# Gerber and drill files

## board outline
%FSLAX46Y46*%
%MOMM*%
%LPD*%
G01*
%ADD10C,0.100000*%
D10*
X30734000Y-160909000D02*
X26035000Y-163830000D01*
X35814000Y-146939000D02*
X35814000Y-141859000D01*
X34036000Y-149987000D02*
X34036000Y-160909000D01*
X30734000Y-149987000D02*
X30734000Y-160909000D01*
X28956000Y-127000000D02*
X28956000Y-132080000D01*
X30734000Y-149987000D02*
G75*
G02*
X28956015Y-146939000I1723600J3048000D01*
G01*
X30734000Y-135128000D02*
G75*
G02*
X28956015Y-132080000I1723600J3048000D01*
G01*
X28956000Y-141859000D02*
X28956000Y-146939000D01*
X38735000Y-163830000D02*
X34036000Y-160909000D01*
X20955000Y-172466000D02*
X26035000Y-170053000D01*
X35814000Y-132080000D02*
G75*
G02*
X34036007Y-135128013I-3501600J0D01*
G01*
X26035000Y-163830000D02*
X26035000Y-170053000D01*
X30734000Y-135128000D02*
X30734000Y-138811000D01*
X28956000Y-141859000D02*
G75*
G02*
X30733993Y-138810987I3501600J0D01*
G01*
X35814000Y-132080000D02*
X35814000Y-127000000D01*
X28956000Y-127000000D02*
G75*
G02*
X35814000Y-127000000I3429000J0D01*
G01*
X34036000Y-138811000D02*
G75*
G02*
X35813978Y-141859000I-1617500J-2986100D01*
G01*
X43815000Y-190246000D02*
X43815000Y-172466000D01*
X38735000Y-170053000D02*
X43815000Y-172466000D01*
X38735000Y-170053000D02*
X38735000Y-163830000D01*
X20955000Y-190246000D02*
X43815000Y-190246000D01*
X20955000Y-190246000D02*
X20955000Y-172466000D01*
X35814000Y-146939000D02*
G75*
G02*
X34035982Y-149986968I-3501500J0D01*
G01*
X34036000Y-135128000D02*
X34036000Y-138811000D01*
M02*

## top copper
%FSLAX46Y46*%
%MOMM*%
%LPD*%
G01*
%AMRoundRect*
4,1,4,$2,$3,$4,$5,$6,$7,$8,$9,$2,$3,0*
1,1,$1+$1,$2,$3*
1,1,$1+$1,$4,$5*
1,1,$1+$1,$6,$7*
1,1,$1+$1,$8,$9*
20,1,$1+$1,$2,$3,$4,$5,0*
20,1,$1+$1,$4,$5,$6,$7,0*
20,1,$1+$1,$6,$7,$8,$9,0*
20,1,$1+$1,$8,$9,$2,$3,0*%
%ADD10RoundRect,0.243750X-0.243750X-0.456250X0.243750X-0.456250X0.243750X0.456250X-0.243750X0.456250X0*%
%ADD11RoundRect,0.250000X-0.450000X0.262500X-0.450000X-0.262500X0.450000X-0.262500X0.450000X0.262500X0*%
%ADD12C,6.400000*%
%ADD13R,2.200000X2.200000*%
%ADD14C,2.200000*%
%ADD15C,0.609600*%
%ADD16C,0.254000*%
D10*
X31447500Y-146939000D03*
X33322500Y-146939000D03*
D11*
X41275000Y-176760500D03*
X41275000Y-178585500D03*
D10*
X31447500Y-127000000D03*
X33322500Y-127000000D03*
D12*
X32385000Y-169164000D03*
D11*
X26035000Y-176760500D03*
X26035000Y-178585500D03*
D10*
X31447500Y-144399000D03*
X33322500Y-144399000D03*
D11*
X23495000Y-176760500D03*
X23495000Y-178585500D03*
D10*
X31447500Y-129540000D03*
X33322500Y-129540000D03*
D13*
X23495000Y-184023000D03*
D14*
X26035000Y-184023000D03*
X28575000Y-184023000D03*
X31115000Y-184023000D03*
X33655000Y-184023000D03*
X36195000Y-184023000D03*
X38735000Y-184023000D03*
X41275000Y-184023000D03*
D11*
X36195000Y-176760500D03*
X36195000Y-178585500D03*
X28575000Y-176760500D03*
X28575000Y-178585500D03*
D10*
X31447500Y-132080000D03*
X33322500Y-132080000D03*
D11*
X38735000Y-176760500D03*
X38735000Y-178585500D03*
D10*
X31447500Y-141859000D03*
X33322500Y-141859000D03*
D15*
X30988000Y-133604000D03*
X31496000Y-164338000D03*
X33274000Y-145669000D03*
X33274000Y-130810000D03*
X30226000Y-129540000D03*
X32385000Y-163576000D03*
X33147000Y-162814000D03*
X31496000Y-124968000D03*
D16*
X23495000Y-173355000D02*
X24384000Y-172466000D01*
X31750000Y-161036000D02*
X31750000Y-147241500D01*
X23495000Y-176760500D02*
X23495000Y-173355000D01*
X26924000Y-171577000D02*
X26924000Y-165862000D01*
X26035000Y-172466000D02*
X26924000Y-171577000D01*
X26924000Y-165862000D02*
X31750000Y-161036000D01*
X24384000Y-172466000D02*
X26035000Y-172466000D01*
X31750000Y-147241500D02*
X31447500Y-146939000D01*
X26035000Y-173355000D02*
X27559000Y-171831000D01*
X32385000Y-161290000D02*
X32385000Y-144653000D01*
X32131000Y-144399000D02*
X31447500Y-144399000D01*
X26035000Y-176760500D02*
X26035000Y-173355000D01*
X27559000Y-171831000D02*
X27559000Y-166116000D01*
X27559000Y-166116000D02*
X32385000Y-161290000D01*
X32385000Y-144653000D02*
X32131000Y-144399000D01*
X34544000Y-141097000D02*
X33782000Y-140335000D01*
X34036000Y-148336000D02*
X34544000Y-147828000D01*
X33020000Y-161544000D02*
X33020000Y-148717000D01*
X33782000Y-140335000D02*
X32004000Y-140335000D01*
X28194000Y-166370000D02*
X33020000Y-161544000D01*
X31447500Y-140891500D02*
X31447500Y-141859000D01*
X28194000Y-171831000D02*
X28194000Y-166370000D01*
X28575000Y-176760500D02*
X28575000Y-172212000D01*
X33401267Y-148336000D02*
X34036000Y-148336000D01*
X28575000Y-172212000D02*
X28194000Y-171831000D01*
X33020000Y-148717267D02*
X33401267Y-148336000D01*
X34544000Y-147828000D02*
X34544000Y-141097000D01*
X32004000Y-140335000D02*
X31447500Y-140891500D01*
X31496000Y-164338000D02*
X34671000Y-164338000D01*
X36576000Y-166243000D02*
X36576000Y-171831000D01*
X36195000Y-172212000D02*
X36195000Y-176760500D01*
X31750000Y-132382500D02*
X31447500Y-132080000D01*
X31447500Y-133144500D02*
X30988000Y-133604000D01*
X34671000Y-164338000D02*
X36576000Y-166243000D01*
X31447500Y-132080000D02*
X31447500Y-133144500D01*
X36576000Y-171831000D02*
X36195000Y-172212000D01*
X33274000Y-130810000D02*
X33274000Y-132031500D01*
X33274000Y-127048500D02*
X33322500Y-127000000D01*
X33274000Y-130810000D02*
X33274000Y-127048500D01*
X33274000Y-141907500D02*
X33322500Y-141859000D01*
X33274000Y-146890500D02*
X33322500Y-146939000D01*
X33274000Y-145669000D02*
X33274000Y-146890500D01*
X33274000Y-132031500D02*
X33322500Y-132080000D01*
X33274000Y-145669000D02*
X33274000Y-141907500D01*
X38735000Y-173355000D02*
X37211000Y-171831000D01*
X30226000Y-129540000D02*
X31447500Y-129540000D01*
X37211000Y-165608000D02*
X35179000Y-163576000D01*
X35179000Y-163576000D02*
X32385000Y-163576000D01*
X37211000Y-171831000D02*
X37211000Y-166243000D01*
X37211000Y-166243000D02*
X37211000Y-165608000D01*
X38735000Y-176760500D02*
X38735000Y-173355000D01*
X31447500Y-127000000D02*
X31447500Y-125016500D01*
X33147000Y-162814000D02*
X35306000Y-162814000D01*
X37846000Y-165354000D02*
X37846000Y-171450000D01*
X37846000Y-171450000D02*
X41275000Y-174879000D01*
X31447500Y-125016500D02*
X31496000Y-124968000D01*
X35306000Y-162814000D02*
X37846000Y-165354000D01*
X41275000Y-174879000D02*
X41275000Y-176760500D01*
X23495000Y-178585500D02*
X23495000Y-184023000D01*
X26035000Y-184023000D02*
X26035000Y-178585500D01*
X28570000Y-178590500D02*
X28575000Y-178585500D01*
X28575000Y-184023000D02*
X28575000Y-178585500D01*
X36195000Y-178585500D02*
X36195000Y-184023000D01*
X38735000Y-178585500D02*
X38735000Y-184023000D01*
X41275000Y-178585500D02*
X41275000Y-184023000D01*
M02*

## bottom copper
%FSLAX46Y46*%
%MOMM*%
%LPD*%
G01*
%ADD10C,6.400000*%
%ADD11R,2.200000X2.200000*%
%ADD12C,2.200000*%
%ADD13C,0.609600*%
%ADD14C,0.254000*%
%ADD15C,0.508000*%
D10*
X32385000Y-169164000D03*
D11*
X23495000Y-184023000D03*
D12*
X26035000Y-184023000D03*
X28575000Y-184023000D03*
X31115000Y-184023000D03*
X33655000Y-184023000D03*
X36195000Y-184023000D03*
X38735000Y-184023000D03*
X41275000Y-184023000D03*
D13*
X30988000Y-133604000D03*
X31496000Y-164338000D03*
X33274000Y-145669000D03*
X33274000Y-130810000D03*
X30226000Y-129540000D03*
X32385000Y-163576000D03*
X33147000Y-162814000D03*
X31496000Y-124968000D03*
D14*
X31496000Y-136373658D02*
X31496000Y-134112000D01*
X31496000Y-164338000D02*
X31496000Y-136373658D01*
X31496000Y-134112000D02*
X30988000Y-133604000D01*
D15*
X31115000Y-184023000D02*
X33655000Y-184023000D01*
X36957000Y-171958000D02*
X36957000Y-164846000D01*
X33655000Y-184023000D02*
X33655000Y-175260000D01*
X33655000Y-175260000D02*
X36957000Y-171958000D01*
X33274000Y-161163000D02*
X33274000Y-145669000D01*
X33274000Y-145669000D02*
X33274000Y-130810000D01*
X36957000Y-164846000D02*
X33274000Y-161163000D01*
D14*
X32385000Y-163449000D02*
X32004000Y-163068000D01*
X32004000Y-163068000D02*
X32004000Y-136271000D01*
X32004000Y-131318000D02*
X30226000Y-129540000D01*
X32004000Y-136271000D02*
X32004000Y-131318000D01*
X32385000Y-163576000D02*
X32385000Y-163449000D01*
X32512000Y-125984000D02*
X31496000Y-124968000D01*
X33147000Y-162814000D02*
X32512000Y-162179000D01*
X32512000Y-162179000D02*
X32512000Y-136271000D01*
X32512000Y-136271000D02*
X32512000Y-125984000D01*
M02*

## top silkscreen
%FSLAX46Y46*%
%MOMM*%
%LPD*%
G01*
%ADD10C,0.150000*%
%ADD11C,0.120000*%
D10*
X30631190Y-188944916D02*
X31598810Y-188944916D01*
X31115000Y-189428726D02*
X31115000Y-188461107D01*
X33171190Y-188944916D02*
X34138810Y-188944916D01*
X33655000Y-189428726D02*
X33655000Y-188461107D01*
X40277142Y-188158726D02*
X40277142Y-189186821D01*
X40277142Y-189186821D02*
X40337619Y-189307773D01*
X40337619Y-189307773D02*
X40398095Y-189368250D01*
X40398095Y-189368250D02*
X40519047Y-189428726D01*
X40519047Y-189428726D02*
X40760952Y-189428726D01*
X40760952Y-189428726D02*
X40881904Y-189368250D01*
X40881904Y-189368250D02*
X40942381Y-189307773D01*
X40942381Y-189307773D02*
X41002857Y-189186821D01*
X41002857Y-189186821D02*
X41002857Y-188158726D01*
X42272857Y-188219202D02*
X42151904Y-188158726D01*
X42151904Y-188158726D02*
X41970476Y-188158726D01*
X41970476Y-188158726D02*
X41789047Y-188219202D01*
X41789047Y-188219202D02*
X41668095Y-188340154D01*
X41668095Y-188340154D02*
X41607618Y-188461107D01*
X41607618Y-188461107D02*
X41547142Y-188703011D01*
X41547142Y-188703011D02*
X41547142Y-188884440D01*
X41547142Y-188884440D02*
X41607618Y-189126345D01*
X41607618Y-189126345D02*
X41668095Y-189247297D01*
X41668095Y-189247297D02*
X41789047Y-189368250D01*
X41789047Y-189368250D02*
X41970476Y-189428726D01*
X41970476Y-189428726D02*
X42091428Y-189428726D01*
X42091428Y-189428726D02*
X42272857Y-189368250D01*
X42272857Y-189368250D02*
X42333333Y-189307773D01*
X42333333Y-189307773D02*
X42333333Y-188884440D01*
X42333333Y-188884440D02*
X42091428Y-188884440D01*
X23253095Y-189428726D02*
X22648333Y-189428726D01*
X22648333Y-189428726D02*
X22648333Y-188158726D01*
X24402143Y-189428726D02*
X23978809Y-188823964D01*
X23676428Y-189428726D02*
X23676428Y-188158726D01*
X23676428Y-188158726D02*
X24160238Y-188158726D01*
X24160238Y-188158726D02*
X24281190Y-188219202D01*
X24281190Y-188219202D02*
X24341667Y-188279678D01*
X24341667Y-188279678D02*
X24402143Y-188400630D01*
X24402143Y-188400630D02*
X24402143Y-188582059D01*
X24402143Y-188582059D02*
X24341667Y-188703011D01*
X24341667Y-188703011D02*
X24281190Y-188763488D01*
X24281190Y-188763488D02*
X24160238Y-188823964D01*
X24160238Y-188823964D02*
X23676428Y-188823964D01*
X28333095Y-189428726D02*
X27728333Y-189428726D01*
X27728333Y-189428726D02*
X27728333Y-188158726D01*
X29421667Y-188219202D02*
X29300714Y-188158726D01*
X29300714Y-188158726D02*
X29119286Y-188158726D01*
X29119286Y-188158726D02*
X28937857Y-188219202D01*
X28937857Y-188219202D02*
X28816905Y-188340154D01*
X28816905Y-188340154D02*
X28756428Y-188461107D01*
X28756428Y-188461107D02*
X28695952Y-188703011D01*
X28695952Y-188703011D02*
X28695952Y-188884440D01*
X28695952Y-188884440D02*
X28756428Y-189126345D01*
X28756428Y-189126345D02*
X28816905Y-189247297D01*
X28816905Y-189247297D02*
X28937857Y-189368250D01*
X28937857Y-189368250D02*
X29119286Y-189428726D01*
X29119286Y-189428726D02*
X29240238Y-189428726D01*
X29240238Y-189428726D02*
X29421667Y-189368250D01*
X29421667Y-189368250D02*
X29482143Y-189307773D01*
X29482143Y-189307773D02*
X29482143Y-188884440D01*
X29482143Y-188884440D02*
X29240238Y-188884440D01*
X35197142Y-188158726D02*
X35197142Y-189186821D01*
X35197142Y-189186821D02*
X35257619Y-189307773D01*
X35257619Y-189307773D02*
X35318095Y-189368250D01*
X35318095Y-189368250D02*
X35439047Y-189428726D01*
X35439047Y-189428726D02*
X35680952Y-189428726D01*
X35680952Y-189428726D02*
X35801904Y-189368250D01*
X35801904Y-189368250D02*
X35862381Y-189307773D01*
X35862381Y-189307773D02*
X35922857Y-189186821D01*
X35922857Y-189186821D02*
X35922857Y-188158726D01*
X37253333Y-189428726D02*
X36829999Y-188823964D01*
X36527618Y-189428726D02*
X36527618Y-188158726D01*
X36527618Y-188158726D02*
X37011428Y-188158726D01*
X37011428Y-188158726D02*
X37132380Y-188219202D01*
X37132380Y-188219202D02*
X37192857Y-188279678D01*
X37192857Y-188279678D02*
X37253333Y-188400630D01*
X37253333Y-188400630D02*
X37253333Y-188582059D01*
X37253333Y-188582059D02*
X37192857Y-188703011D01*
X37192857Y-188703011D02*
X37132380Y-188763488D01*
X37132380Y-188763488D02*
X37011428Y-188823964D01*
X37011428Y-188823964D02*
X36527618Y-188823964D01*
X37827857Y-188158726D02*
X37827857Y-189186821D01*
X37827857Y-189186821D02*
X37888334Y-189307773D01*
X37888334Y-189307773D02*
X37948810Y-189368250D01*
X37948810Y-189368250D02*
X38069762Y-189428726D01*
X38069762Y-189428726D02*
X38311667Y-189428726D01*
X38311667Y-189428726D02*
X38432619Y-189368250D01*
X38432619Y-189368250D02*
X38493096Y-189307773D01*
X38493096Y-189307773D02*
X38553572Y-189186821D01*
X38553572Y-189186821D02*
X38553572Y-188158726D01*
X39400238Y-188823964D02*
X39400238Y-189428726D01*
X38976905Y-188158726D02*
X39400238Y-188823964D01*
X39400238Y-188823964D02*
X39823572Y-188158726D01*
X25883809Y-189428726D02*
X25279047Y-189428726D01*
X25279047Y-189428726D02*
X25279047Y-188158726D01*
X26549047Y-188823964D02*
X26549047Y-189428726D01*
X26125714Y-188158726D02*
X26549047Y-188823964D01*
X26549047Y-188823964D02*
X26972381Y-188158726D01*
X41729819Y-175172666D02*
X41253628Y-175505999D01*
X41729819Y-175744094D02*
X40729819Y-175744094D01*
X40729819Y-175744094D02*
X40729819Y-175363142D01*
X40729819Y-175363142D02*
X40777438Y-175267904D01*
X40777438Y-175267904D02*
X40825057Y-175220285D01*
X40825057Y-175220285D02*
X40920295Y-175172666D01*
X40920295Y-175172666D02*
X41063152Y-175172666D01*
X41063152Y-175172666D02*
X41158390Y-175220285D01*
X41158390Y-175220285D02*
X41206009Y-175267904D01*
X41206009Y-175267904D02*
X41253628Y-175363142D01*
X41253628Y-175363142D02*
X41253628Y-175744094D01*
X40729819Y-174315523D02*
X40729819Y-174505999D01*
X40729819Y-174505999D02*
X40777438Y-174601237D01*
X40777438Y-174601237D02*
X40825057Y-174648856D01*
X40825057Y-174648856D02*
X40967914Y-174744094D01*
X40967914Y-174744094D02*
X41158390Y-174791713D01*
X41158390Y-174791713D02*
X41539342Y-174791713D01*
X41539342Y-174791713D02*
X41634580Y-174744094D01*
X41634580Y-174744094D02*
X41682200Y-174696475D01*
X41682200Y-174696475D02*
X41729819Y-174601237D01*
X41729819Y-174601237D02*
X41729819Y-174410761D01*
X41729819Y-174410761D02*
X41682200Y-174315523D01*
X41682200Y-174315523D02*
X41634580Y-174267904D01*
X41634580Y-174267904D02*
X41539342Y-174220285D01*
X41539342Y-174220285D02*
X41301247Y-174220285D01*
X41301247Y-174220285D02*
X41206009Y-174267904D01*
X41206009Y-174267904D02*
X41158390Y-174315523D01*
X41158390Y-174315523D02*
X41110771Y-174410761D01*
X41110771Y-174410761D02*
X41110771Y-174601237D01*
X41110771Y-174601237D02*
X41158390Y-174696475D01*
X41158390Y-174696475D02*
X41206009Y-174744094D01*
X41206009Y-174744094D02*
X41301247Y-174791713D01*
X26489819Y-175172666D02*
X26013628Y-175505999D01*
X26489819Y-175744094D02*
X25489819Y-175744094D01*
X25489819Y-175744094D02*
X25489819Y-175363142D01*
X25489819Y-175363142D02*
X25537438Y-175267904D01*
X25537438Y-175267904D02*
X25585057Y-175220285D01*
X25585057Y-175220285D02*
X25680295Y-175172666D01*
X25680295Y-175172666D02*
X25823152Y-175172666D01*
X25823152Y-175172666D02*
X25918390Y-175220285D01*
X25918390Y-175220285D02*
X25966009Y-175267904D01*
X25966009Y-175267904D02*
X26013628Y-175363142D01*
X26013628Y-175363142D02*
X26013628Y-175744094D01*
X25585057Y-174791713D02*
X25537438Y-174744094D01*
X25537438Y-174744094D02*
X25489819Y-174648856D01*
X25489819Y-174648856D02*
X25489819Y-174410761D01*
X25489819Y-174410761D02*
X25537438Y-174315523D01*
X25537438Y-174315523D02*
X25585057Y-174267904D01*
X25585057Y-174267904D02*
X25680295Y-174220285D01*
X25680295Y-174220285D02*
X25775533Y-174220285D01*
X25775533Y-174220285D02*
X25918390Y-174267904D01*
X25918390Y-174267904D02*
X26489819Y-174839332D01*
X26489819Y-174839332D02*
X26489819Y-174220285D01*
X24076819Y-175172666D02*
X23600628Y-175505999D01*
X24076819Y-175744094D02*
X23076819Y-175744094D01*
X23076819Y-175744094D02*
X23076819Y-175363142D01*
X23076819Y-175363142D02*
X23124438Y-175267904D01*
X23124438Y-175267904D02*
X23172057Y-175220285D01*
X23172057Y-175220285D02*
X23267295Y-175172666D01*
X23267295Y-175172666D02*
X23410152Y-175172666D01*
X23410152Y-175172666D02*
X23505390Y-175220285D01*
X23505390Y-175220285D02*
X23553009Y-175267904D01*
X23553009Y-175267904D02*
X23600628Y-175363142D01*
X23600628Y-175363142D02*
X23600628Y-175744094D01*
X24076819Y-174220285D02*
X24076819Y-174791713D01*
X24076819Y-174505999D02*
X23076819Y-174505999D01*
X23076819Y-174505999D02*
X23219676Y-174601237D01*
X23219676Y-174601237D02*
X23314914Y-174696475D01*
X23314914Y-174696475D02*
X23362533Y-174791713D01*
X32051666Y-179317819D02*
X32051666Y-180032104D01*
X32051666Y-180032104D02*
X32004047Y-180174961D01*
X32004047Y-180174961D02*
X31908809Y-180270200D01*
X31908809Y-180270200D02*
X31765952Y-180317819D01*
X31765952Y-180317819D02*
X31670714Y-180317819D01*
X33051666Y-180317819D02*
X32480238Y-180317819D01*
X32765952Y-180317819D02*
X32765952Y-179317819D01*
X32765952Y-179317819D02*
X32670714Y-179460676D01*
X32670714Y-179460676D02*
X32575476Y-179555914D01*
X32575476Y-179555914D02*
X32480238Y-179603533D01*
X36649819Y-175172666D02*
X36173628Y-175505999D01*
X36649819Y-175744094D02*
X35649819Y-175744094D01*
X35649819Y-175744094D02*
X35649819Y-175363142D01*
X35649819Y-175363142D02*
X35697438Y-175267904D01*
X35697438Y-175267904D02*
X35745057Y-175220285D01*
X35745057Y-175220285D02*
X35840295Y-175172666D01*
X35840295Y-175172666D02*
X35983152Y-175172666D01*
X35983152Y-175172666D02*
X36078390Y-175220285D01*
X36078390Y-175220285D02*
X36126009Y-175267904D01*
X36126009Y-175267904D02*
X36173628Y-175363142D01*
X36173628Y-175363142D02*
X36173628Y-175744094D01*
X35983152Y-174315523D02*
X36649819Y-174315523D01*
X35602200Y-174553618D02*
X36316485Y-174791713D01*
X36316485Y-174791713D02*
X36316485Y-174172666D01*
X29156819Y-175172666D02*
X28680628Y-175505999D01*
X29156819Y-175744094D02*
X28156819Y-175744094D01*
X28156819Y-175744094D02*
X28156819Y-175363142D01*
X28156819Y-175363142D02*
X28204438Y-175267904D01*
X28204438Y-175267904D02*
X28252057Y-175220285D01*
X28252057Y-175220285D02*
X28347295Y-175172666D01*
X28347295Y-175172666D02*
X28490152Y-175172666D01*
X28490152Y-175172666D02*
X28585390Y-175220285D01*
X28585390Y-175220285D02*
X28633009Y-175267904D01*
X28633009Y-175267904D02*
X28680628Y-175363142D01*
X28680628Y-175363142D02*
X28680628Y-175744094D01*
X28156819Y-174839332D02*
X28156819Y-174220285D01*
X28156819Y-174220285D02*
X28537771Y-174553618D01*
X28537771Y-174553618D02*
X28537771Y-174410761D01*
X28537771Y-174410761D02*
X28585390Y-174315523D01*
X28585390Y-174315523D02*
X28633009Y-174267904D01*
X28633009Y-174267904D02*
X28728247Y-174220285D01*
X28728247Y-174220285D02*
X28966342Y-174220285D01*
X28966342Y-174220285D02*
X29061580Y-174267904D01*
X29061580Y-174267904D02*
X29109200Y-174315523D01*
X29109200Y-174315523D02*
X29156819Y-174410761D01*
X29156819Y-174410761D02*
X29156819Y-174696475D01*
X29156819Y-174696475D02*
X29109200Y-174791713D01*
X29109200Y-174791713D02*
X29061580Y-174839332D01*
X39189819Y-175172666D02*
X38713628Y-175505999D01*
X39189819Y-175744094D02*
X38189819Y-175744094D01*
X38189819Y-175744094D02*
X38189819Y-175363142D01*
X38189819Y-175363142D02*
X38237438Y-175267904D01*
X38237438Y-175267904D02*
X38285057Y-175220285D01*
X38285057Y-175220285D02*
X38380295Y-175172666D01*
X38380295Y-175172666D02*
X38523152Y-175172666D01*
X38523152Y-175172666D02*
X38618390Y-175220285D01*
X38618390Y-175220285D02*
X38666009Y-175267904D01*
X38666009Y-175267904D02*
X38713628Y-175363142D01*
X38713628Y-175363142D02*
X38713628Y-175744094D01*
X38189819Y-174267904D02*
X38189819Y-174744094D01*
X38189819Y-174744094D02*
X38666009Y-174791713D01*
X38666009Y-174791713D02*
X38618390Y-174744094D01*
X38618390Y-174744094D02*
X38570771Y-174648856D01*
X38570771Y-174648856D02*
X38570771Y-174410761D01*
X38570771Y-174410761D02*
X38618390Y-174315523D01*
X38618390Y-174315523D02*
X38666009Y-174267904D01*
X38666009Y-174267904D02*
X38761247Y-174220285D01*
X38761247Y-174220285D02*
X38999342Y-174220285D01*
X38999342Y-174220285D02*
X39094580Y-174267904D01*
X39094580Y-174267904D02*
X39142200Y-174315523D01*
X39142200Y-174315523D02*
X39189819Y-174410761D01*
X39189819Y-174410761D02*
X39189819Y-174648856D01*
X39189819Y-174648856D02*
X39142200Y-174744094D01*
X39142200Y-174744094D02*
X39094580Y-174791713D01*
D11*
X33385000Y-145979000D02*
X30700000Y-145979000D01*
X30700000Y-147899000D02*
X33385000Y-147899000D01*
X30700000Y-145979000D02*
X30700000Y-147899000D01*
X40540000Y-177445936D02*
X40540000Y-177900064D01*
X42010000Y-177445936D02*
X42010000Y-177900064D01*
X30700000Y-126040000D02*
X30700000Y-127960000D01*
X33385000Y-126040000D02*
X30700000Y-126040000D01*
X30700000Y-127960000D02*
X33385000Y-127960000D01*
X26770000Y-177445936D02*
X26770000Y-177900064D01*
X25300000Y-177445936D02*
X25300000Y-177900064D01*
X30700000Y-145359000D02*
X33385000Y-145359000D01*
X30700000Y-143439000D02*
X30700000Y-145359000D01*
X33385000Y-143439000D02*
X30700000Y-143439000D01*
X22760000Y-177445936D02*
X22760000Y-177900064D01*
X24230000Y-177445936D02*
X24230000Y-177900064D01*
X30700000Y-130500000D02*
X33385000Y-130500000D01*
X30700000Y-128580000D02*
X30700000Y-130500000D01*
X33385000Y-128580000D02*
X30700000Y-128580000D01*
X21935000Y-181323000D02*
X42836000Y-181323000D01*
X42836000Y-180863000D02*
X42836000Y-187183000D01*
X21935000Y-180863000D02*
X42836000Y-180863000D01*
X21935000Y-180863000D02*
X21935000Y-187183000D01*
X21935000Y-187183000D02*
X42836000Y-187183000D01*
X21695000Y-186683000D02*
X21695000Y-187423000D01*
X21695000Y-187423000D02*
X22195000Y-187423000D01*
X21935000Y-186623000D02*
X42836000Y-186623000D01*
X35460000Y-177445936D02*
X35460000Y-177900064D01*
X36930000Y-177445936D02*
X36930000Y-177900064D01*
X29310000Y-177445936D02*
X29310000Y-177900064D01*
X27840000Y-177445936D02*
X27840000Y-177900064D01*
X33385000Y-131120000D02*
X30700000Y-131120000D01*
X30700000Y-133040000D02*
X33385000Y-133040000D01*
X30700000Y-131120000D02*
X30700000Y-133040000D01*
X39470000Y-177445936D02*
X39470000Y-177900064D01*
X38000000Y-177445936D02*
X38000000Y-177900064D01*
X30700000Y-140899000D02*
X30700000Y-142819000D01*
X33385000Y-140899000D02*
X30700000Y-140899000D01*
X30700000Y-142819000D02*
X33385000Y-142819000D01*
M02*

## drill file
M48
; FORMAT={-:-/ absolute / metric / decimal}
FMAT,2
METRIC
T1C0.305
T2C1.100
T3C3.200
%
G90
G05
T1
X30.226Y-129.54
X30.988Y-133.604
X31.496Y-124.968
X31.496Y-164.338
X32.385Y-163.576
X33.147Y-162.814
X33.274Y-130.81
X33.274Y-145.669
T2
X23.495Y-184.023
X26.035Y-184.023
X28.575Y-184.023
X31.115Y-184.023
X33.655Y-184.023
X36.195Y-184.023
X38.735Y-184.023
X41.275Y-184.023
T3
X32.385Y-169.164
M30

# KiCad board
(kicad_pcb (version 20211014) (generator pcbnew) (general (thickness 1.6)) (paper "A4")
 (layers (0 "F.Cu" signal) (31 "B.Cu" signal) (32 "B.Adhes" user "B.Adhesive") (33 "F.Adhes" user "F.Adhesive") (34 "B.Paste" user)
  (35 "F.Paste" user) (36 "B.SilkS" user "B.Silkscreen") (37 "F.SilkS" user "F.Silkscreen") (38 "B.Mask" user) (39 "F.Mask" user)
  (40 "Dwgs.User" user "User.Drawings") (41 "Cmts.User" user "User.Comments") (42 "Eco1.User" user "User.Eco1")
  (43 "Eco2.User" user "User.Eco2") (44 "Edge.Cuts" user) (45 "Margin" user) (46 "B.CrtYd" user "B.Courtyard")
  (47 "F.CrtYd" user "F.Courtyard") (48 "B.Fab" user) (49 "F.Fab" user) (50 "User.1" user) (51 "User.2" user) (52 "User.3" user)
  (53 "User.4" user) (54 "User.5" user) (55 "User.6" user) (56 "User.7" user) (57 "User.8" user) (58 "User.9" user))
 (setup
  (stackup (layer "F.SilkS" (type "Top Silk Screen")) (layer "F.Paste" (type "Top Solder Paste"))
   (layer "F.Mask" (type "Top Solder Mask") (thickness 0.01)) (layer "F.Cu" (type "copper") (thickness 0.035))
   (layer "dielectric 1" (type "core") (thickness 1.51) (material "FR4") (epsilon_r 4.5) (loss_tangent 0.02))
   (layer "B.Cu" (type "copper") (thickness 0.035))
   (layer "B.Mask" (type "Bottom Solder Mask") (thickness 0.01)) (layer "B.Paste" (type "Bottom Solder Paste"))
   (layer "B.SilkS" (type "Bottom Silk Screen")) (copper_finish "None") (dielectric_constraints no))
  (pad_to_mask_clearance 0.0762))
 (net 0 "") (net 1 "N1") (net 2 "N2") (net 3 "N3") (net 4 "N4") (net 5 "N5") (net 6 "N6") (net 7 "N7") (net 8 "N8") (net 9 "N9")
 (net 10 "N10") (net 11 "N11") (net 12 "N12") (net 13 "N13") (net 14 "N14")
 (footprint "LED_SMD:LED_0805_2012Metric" (layer "F.Cu") (at 32.385 146.939)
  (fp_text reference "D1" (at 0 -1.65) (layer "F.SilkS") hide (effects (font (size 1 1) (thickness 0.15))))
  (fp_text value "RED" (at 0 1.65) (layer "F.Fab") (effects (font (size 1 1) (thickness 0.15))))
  (fp_line (start 1 -0.96) (end -1.685 -0.96) (layer "F.SilkS") (width 0.12))
  (fp_line (start -1.685 0.96) (end 1 0.96) (layer "F.SilkS") (width 0.12))
  (fp_line (start -1.685 -0.96) (end -1.685 0.96) (layer "F.SilkS") (width 0.12))
  (pad "1" smd roundrect (at -0.9375 0) (size 0.975 1.4) (layers "F.Cu" "F.Paste" "F.Mask") (roundrect_rratio 0.25) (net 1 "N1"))
  (pad "2" smd roundrect (at 0.9375 0) (size 0.975 1.4) (layers "F.Cu" "F.Paste" "F.Mask") (roundrect_rratio 0.25) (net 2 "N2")))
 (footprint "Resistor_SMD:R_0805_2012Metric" (layer "F.Cu") (at 41.275 177.673 -90)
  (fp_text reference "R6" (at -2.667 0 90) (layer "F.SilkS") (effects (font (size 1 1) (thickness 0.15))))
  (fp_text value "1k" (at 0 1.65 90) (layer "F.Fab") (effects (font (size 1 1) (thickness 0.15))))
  (fp_line (start -0.227064 0.735) (end 0.227064 0.735) (layer "F.SilkS") (width 0.12))
  (fp_line (start -0.227064 -0.735) (end 0.227064 -0.735) (layer "F.SilkS") (width 0.12))
  (pad "1" smd roundrect (at -0.9125 0 270) (size 1.025 1.4) (layers "F.Cu" "F.Paste" "F.Mask") (roundrect_rratio 0.243902) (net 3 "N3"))
  (pad "2" smd roundrect (at 0.9125 0 270) (size 1.025 1.4) (layers "F.Cu" "F.Paste" "F.Mask") (roundrect_rratio 0.243902) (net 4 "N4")))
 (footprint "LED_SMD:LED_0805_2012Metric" (layer "F.Cu") (at 32.385 127)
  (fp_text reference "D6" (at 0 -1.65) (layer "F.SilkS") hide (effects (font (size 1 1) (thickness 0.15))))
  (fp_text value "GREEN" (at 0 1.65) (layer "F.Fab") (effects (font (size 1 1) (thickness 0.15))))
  (fp_line (start -1.685 -0.96) (end -1.685 0.96) (layer "F.SilkS") (width 0.12))
  (fp_line (start 1 -0.96) (end -1.685 -0.96) (layer "F.SilkS") (width 0.12))
  (fp_line (start -1.685 0.96) (end 1 0.96) (layer "F.SilkS") (width 0.12))
  (pad "1" smd roundrect (at -0.9375 0) (size 0.975 1.4) (layers "F.Cu" "F.Paste" "F.Mask") (roundrect_rratio 0.25) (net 3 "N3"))
  (pad "2" smd roundrect (at 0.9375 0) (size 0.975 1.4) (layers "F.Cu" "F.Paste" "F.Mask") (roundrect_rratio 0.25) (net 2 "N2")))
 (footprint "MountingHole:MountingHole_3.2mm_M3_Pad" (layer "F.Cu") (at 32.385 169.164) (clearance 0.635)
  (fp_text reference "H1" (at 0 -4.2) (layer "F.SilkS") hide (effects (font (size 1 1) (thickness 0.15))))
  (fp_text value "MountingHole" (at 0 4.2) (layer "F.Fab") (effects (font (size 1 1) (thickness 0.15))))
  (pad "1" thru_hole circle (at 0 0) (size 6.4 6.4) (drill 3.2) (layers *.Cu *.Mask) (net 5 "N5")))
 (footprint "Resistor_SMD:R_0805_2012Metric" (layer "F.Cu") (at 26.035 177.673 -90)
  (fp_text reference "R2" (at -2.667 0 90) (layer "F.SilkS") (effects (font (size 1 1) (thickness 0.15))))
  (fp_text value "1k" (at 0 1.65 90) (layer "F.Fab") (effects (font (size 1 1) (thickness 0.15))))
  (fp_line (start -0.227064 -0.735) (end 0.227064 -0.735) (layer "F.SilkS") (width 0.12))
  (fp_line (start -0.227064 0.735) (end 0.227064 0.735) (layer "F.SilkS") (width 0.12))
  (pad "1" smd roundrect (at -0.9125 0 270) (size 1.025 1.4) (layers "F.Cu" "F.Paste" "F.Mask") (roundrect_rratio 0.243902) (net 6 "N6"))
  (pad "2" smd roundrect (at 0.9125 0 270) (size 1.025 1.4) (layers "F.Cu" "F.Paste" "F.Mask") (roundrect_rratio 0.243902) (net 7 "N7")))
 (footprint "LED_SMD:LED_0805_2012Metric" (layer "F.Cu") (at 32.385 144.399)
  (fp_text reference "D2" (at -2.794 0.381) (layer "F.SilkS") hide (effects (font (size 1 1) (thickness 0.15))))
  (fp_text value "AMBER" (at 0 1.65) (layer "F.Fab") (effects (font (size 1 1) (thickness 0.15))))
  (fp_line (start -1.685 0.96) (end 1 0.96) (layer "F.SilkS") (width 0.12))
  (fp_line (start -1.685 -0.96) (end -1.685 0.96) (layer "F.SilkS") (width 0.12))
  (fp_line (start 1 -0.96) (end -1.685 -0.96) (layer "F.SilkS") (width 0.12))
  (pad "1" smd roundrect (at -0.9375 0) (size 0.975 1.4) (layers "F.Cu" "F.Paste" "F.Mask") (roundrect_rratio 0.25) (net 6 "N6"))
  (pad "2" smd roundrect (at 0.9375 0) (size 0.975 1.4) (layers "F.Cu" "F.Paste" "F.Mask") (roundrect_rratio 0.25) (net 2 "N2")))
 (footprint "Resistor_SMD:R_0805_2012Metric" (layer "F.Cu") (at 23.495 177.673 -90)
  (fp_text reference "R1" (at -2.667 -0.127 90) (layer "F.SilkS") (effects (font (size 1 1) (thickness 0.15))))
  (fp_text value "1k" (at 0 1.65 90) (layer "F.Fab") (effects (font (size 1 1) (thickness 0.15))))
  (fp_line (start -0.227064 0.735) (end 0.227064 0.735) (layer "F.SilkS") (width 0.12))
  (fp_line (start -0.227064 -0.735) (end 0.227064 -0.735) (layer "F.SilkS") (width 0.12))
  (pad "1" smd roundrect (at -0.9125 0 270) (size 1.025 1.4) (layers "F.Cu" "F.Paste" "F.Mask") (roundrect_rratio 0.243902) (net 1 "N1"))
  (pad "2" smd roundrect (at 0.9125 0 270) (size 1.025 1.4) (layers "F.Cu" "F.Paste" "F.Mask") (roundrect_rratio 0.243902) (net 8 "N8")))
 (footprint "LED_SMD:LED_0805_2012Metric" (layer "F.Cu") (at 32.385 129.54)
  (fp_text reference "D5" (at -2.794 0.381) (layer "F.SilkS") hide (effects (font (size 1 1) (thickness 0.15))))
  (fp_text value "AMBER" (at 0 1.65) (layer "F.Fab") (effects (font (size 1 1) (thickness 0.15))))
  (fp_line (start -1.685 0.96) (end 1 0.96) (layer "F.SilkS") (width 0.12))
  (fp_line (start -1.685 -0.96) (end -1.685 0.96) (layer "F.SilkS") (width 0.12))
  (fp_line (start 1 -0.96) (end -1.685 -0.96) (layer "F.SilkS") (width 0.12))
  (pad "1" smd roundrect (at -0.9375 0) (size 0.975 1.4) (layers "F.Cu" "F.Paste" "F.Mask") (roundrect_rratio 0.25) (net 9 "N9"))
  (pad "2" smd roundrect (at 0.9375 0) (size 0.975 1.4) (layers "F.Cu" "F.Paste" "F.Mask") (roundrect_rratio 0.25) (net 2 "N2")))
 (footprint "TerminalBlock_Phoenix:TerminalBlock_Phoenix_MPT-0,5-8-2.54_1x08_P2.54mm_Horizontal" (layer "F.Cu") (at 23.495 184.023)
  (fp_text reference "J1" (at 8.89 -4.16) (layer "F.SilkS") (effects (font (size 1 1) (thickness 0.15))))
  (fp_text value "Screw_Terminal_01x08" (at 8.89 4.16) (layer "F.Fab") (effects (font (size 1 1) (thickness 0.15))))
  (fp_line (start -1.56 -2.7) (end 19.341 -2.7) (layer "F.SilkS") (width 0.12))
  (fp_line (start 19.341 -3.16) (end 19.341 3.16) (layer "F.SilkS") (width 0.12))
  (fp_line (start -1.56 -3.16) (end 19.341 -3.16) (layer "F.SilkS") (width 0.12))
  (fp_line (start -1.56 -3.16) (end -1.56 3.16) (layer "F.SilkS") (width 0.12))
  (fp_line (start -1.56 3.16) (end 19.341 3.16) (layer "F.SilkS") (width 0.12))
  (fp_line (start -1.8 2.66) (end -1.8 3.4) (layer "F.SilkS") (width 0.12))
  (fp_line (start -1.8 3.4) (end -1.3 3.4) (layer "F.SilkS") (width 0.12))
  (fp_line (start -1.56 2.6) (end 19.341 2.6) (layer "F.SilkS") (width 0.12))
  (pad "1" thru_hole rect (at 0 0) (size 2.2 2.2) (drill 1.1) (layers F&B.Cu *.Mask) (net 8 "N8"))
  (pad "2" thru_hole circle (at 2.54 0) (size 2.2 2.2) (drill 1.1) (layers F&B.Cu *.Mask) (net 7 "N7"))
  (pad "3" thru_hole circle (at 5.08 0) (size 2.2 2.2) (drill 1.1) (layers F&B.Cu *.Mask) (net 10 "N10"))
  (pad "4" thru_hole circle (at 7.62 0) (size 2.2 2.2) (drill 1.1) (layers F&B.Cu *.Mask) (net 2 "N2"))
  (pad "5" thru_hole circle (at 10.16 0) (size 2.2 2.2) (drill 1.1) (layers F&B.Cu *.Mask) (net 2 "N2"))
  (pad "6" thru_hole circle (at 12.7 0) (size 2.2 2.2) (drill 1.1) (layers F&B.Cu *.Mask) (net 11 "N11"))
  (pad "7" thru_hole circle (at 15.24 0) (size 2.2 2.2) (drill 1.1) (layers F&B.Cu *.Mask) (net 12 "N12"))
  (pad "8" thru_hole circle (at 17.78 0) (size 2.2 2.2) (drill 1.1) (layers F&B.Cu *.Mask) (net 4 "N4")))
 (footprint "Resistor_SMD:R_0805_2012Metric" (layer "F.Cu") (at 36.195 177.673 -90)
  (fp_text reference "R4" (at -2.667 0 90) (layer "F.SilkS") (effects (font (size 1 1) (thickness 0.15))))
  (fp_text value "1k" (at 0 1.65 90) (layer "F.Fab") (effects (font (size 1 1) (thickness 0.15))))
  (fp_line (start -0.227064 0.735) (end 0.227064 0.735) (layer "F.SilkS") (width 0.12))
  (fp_line (start -0.227064 -0.735) (end 0.227064 -0.735) (layer "F.SilkS") (width 0.12))
  (pad "1" smd roundrect (at -0.9125 0 270) (size 1.025 1.4) (layers "F.Cu" "F.Paste" "F.Mask") (roundrect_rratio 0.243902) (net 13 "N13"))
  (pad "2" smd roundrect (at 0.9125 0 270) (size 1.025 1.4) (layers "F.Cu" "F.Paste" "F.Mask") (roundrect_rratio 0.243902) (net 11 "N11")))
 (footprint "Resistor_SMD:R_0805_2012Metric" (layer "F.Cu") (at 28.575 177.673 -90)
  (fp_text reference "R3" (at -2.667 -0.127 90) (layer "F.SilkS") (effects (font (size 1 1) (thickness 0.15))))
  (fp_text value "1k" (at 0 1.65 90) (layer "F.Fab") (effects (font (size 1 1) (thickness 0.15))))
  (fp_line (start -0.227064 -0.735) (end 0.227064 -0.735) (layer "F.SilkS") (width 0.12))
  (fp_line (start -0.227064 0.735) (end 0.227064 0.735) (layer "F.SilkS") (width 0.12))
  (pad "1" smd roundrect (at -0.9125 0 270) (size 1.025 1.4) (layers "F.Cu" "F.Paste" "F.Mask") (roundrect_rratio 0.243902) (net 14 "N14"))
  (pad "2" smd roundrect (at 0.9125 0 270) (size 1.025 1.4) (layers "F.Cu" "F.Paste" "F.Mask") (roundrect_rratio 0.243902) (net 10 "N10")))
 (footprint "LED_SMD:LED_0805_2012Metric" (layer "F.Cu") (at 32.385 132.08)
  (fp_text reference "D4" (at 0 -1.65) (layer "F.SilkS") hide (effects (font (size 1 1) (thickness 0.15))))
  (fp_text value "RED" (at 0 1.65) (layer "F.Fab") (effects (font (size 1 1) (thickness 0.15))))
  (fp_line (start 1 -0.96) (end -1.685 -0.96) (layer "F.SilkS") (width 0.12))
  (fp_line (start -1.685 0.96) (end 1 0.96) (layer "F.SilkS") (width 0.12))
  (fp_line (start -1.685 -0.96) (end -1.685 0.96) (layer "F.SilkS") (width 0.12))
  (pad "1" smd roundrect (at -0.9375 0) (size 0.975 1.4) (layers "F.Cu" "F.Paste" "F.Mask") (roundrect_rratio 0.25) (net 13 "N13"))
  (pad "2" smd roundrect (at 0.9375 0) (size 0.975 1.4) (layers "F.Cu" "F.Paste" "F.Mask") (roundrect_rratio 0.25) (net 2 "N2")))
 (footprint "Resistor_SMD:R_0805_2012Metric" (layer "F.Cu") (at 38.735 177.673 -90)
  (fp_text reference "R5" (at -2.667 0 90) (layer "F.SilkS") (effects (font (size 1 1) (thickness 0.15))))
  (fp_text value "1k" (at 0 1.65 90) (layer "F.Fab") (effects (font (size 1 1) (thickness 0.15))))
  (fp_line (start -0.227064 -0.735) (end 0.227064 -0.735) (layer "F.SilkS") (width 0.12))
  (fp_line (start -0.227064 0.735) (end 0.227064 0.735) (layer "F.SilkS") (width 0.12))
  (pad "1" smd roundrect (at -0.9125 0 270) (size 1.025 1.4) (layers "F.Cu" "F.Paste" "F.Mask") (roundrect_rratio 0.243902) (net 9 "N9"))
  (pad "2" smd roundrect (at 0.9125 0 270) (size 1.025 1.4) (layers "F.Cu" "F.Paste" "F.Mask") (roundrect_rratio 0.243902) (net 12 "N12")))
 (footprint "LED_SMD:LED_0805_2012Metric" (layer "F.Cu") (at 32.385 141.859)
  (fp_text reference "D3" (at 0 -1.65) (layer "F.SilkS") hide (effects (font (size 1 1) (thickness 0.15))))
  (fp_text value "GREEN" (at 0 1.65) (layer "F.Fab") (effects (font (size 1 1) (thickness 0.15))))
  (fp_line (start -1.685 -0.96) (end -1.685 0.96) (layer "F.SilkS") (width 0.12))
  (fp_line (start 1 -0.96) (end -1.685 -0.96) (layer "F.SilkS") (width 0.12))
  (fp_line (start -1.685 0.96) (end 1 0.96) (layer "F.SilkS") (width 0.12))
  (pad "1" smd roundrect (at -0.9375 0) (size 0.975 1.4) (layers "F.Cu" "F.Paste" "F.Mask") (roundrect_rratio 0.25) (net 14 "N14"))
  (pad "2" smd roundrect (at 0.9375 0) (size 0.975 1.4) (layers "F.Cu" "F.Paste" "F.Mask") (roundrect_rratio 0.25) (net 2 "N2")))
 (gr_line (start 30.734 160.909) (end 26.035 163.83) (layer "Edge.Cuts") (width 0.1))
 (gr_line (start 35.814 146.939) (end 35.814 141.859) (layer "Edge.Cuts") (width 0.1))
 (gr_line (start 34.036 149.987) (end 34.036 160.909) (layer "Edge.Cuts") (width 0.1))
 (gr_line (start 30.734 149.987) (end 30.734 160.909) (layer "Edge.Cuts") (width 0.1))
 (gr_line (start 28.956 127) (end 28.956 132.08) (layer "Edge.Cuts") (width 0.1))
 (gr_arc (start 30.734 149.987) (mid 29.432998 148.703337) (end 28.956 146.939) (layer "Edge.Cuts") (width 0.1))
 (gr_arc (start 30.734 135.128) (mid 29.432997 133.844335) (end 28.956 132.08) (layer "Edge.Cuts") (width 0.1))
 (gr_line (start 28.956 141.859) (end 28.956 146.939) (layer "Edge.Cuts") (width 0.1))
 (gr_line (start 38.735 163.83) (end 34.036 160.909) (layer "Edge.Cuts") (width 0.1))
 (gr_line (start 20.955 172.466) (end 26.035 170.053) (layer "Edge.Cuts") (width 0.1))
 (gr_arc (start 35.814 132.08) (mid 35.337015 133.844342) (end 34.036 135.128) (layer "Edge.Cuts") (width 0.1))
 (gr_line (start 26.035 163.83) (end 26.035 170.053) (layer "Edge.Cuts") (width 0.1))
 (gr_line (start 30.734 135.128) (end 30.734 138.811) (layer "Edge.Cuts") (width 0.1))
 (gr_arc (start 28.956 141.859) (mid 29.432988 140.09466) (end 30.734 138.811) (layer "Edge.Cuts") (width 0.1))
 (gr_line (start 35.814 132.08) (end 35.814 127) (layer "Edge.Cuts") (width 0.1))
 (gr_arc (start 28.956 127) (mid 32.385 123.571) (end 35.814 127) (layer "Edge.Cuts") (width 0.1))
 (gr_arc (start 34.036 138.811) (mid 35.351951 140.085945) (end 35.814 141.859) (layer "Edge.Cuts") (width 0.1))
 (gr_line (start 43.815 190.246) (end 43.815 172.466) (layer "Edge.Cuts") (width 0.1))
 (gr_line (start 38.735 170.053) (end 43.815 172.466) (layer "Edge.Cuts") (width 0.1))
 (gr_line (start 38.735 170.053) (end 38.735 163.83) (layer "Edge.Cuts") (width 0.1))
 (gr_line locked (start 20.955 190.246) (end 43.815 190.246) (layer "Edge.Cuts") (width 0.1))
 (gr_line (start 20.955 190.246) (end 20.955 172.466) (layer "Edge.Cuts") (width 0.1))
 (gr_arc (start 35.814 146.939) (mid 35.337014 148.703344) (end 34.036 149.987) (layer "Edge.Cuts") (width 0.1))
 (gr_line (start 34.036 135.128) (end 34.036 138.811) (layer "Edge.Cuts") (width 0.1))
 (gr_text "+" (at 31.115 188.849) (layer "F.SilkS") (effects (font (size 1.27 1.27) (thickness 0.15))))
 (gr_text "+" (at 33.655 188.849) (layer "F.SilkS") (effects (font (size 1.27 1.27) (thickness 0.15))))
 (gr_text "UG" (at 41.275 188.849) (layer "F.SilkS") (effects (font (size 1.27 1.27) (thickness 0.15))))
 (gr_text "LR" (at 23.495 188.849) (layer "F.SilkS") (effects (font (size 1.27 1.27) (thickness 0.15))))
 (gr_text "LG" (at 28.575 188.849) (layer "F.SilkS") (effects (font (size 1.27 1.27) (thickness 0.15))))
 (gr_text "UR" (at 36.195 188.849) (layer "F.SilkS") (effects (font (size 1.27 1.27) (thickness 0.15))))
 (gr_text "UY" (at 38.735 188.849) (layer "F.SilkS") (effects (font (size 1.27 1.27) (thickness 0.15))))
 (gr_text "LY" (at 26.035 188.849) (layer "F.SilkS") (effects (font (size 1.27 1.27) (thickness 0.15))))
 (segment (start 23.495 173.355) (end 24.384 172.466) (width 0.254) (layer "F.Cu") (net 1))
 (segment (start 31.75 161.036) (end 31.75 147.2415) (width 0.254) (layer "F.Cu") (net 1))
 (segment (start 23.495 176.7605) (end 23.495 173.355) (width 0.254) (layer "F.Cu") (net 1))
 (segment (start 26.924 171.577) (end 26.924 165.862) (width 0.254) (layer "F.Cu") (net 1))
 (segment (start 26.035 172.466) (end 26.924 171.577) (width 0.254) (layer "F.Cu") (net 1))
 (segment (start 26.924 165.862) (end 31.75 161.036) (width 0.254) (layer "F.Cu") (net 1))
 (segment (start 24.384 172.466) (end 26.035 172.466) (width 0.254) (layer "F.Cu") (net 1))
 (segment (start 31.75 147.2415) (end 31.4475 146.939) (width 0.254) (layer "F.Cu") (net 1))
 (segment (start 26.035 173.355) (end 27.559 171.831) (width 0.254) (layer "F.Cu") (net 6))
 (segment (start 32.385 161.29) (end 32.385 144.653) (width 0.254) (layer "F.Cu") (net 6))
 (segment (start 32.131 144.399) (end 31.4475 144.399) (width 0.254) (layer "F.Cu") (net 6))
 (segment (start 26.035 176.7605) (end 26.035 173.355) (width 0.254) (layer "F.Cu") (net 6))
 (segment (start 27.559 171.831) (end 27.559 166.116) (width 0.254) (layer "F.Cu") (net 6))
 (segment (start 27.559 166.116) (end 32.385 161.29) (width 0.254) (layer "F.Cu") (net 6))
 (segment (start 32.385 144.653) (end 32.131 144.399) (width 0.254) (layer "F.Cu") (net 6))
 (segment (start 34.544 141.097) (end 33.782 140.335) (width 0.254) (layer "F.Cu") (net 14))
 (segment (start 34.036 148.336) (end 34.544 147.828) (width 0.254) (layer "F.Cu") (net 14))
 (segment (start 33.02 161.544) (end 33.02 148.717) (width 0.254) (layer "F.Cu") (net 14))
 (segment (start 33.782 140.335) (end 32.004 140.335) (width 0.254) (layer "F.Cu") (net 14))
 (segment (start 28.194 166.37) (end 33.02 161.544) (width 0.254) (layer "F.Cu") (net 14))
 (segment (start 31.4475 140.8915) (end 31.4475 141.859) (width 0.254) (layer "F.Cu") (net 14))
 (segment (start 28.194 171.831) (end 28.194 166.37) (width 0.254) (layer "F.Cu") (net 14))
 (segment (start 28.575 176.7605) (end 28.575 172.212) (width 0.254) (layer "F.Cu") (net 14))
 (segment (start 33.401267 148.336) (end 34.036 148.336) (width 0.254) (layer "F.Cu") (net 14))
 (segment (start 28.575 172.212) (end 28.194 171.831) (width 0.254) (layer "F.Cu") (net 14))
 (segment (start 33.02 148.717267) (end 33.401267 148.336) (width 0.254) (layer "F.Cu") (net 14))
 (segment (start 34.544 147.828) (end 34.544 141.097) (width 0.254) (layer "F.Cu") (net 14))
 (segment (start 32.004 140.335) (end 31.4475 140.8915) (width 0.254) (layer "F.Cu") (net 14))
 (segment (start 31.496 164.338) (end 34.671 164.338) (width 0.254) (layer "F.Cu") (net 13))
 (segment (start 36.576 166.243) (end 36.576 171.831) (width 0.254) (layer "F.Cu") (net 13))
 (segment (start 36.195 172.212) (end 36.195 176.7605) (width 0.254) (layer "F.Cu") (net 13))
 (segment (start 31.75 132.3825) (end 31.4475 132.08) (width 0.254) (layer "F.Cu") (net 13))
 (segment (start 31.4475 133.1445) (end 30.988 133.604) (width 0.254) (layer "F.Cu") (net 13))
 (segment (start 34.671 164.338) (end 36.576 166.243) (width 0.254) (layer "F.Cu") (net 13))
 (segment (start 31.4475 132.08) (end 31.4475 133.1445) (width 0.254) (layer "F.Cu") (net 13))
 (segment (start 36.576 171.831) (end 36.195 172.212) (width 0.254) (layer "F.Cu") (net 13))
 (via (at 30.988 133.604) (size 0.6096) (drill 0.3048) (layers "F.Cu" "B.Cu") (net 13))
 (via (at 31.496 164.338) (size 0.6096) (drill 0.3048) (layers "F.Cu" "B.Cu") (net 13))
 (segment (start 31.496 136.373658) (end 31.496 134.112) (width 0.254) (layer "B.Cu") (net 13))
 (segment (start 31.496 164.338) (end 31.496 136.373658) (width 0.254) (layer "B.Cu") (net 13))
 (segment (start 31.496 134.112) (end 30.988 133.604) (width 0.254) (layer "B.Cu") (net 13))
 (segment (start 33.274 130.81) (end 33.274 132.0315) (width 0.254) (layer "F.Cu") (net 2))
 (segment (start 33.274 127.0485) (end 33.3225 127) (width 0.254) (layer "F.Cu") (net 2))
 (segment (start 33.274 130.81) (end 33.274 127.0485) (width 0.254) (layer "F.Cu") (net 2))
 (segment (start 33.274 141.9075) (end 33.3225 141.859) (width 0.254) (layer "F.Cu") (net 2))
 (segment (start 33.274 146.8905) (end 33.3225 146.939) (width 0.254) (layer "F.Cu") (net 2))
 (segment (start 33.274 145.669) (end 33.274 146.8905) (width 0.254) (layer "F.Cu") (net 2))
 (segment (start 33.274 132.0315) (end 33.3225 132.08) (width 0.254) (layer "F.Cu") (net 2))
 (segment (start 33.274 145.669) (end 33.274 141.9075) (width 0.254) (layer "F.Cu") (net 2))
 (via (at 33.274 145.669) (size 0.6096) (drill 0.3048) (layers "F.Cu" "B.Cu") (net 2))
 (via (at 33.274 130.81) (size 0.6096) (drill 0.3048) (layers "F.Cu" "B.Cu") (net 2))
 (segment (start 31.115 184.023) (end 33.655 184.023) (width 0.508) (layer "B.Cu") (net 2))
 (segment (start 36.957 171.958) (end 36.957 164.846) (width 0.508) (layer "B.Cu") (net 2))
 (segment (start 33.655 184.023) (end 33.655 175.26) (width 0.508) (layer "B.Cu") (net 2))
 (segment (start 33.655 175.26) (end 36.957 171.958) (width 0.508) (layer "B.Cu") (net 2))
 (segment (start 33.274 161.163) (end 33.274 145.669) (width 0.508) (layer "B.Cu") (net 2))
 (segment (start 33.274 145.669) (end 33.274 130.81) (width 0.508) (layer "B.Cu") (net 2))
 (segment (start 36.957 164.846) (end 33.274 161.163) (width 0.508) (layer "B.Cu") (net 2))
 (segment (start 38.735 173.355) (end 37.211 171.831) (width 0.254) (layer "F.Cu") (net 9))
 (segment (start 30.226 129.54) (end 31.4475 129.54) (width 0.254) (layer "F.Cu") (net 9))
 (segment (start 37.211 165.608) (end 35.179 163.576) (width 0.254) (layer "F.Cu") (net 9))
 (segment (start 35.179 163.576) (end 32.385 163.576) (width 0.254) (layer "F.Cu") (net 9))
 (segment (start 37.211 171.831) (end 37.211 166.243) (width 0.254) (layer "F.Cu") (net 9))
 (segment (start 37.211 166.243) (end 37.211 165.608) (width 0.254) (layer "F.Cu") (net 9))
 (segment (start 38.735 176.7605) (end 38.735 173.355) (width 0.254) (layer "F.Cu") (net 9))
 (via (at 30.226 129.54) (size 0.6096) (drill 0.3048) (layers "F.Cu" "B.Cu") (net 9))
 (via (at 32.385 163.576) (size 0.6096) (drill 0.3048) (layers "F.Cu" "B.Cu") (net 9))
 (segment (start 32.385 163.449) (end 32.004 163.068) (width 0.254) (layer "B.Cu") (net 9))
 (segment (start 32.004 163.068) (end 32.004 136.271) (width 0.254) (layer "B.Cu") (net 9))
 (segment (start 32.004 131.318) (end 30.226 129.54) (width 0.254) (layer "B.Cu") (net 9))
 (segment (start 32.004 136.271) (end 32.004 131.318) (width 0.254) (layer "B.Cu") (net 9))
 (segment (start 32.385 163.576) (end 32.385 163.449) (width 0.254) (layer "B.Cu") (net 9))
 (segment (start 31.4475 127) (end 31.4475 125.0165) (width 0.254) (layer "F.Cu") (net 3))
 (segment (start 33.147 162.814) (end 35.306 162.814) (width 0.254) (layer "F.Cu") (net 3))
 (segment (start 37.846 165.354) (end 37.846 171.45) (width 0.254) (layer "F.Cu") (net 3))
 (segment (start 37.846 171.45) (end 41.275 174.879) (width 0.254) (layer "F.Cu") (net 3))
 (segment (start 31.4475 125.0165) (end 31.496 124.968) (width 0.254) (layer "F.Cu") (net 3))
 (segment (start 35.306 162.814) (end 37.846 165.354) (width 0.254) (layer "F.Cu") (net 3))
 (segment (start 41.275 174.879) (end 41.275 176.7605) (width 0.254) (layer "F.Cu") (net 3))
 (via (at 33.147 162.814) (size 0.6096) (drill 0.3048) (layers "F.Cu" "B.Cu") (free) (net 3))
 (via (at 31.496 124.968) (size 0.6096) (drill 0.3048) (layers "F.Cu" "B.Cu") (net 3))
 (segment (start 32.512 125.984) (end 31.496 124.968) (width 0.254) (layer "B.Cu") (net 3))
 (segment (start 33.147 162.814) (end 32.512 162.179) (width 0.254) (layer "B.Cu") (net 3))
 (segment (start 32.512 162.179) (end 32.512 136.271) (width 0.254) (layer "B.Cu") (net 3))
 (segment (start 32.512 136.271) (end 32.512 125.984) (width 0.254) (layer "B.Cu") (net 3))
 (segment (start 23.495 178.5855) (end 23.495 184.023) (width 0.254) (layer "F.Cu") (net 8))
 (segment (start 26.035 184.023) (end 26.035 178.5855) (width 0.254) (layer "F.Cu") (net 7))
 (segment (start 28.57 178.5905) (end 28.575 178.5855) (width 0.254) (layer "F.Cu") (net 10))
 (segment (start 28.575 184.023) (end 28.575 178.5855) (width 0.254) (layer "F.Cu") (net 10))
 (segment (start 36.195 178.5855) (end 36.195 184.023) (width 0.254) (layer "F.Cu") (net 11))
 (segment (start 38.735 178.5855) (end 38.735 184.023) (width 0.254) (layer "F.Cu") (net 12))
 (segment (start 41.275 178.5855) (end 41.275 184.023) (width 0.254) (layer "F.Cu") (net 4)))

